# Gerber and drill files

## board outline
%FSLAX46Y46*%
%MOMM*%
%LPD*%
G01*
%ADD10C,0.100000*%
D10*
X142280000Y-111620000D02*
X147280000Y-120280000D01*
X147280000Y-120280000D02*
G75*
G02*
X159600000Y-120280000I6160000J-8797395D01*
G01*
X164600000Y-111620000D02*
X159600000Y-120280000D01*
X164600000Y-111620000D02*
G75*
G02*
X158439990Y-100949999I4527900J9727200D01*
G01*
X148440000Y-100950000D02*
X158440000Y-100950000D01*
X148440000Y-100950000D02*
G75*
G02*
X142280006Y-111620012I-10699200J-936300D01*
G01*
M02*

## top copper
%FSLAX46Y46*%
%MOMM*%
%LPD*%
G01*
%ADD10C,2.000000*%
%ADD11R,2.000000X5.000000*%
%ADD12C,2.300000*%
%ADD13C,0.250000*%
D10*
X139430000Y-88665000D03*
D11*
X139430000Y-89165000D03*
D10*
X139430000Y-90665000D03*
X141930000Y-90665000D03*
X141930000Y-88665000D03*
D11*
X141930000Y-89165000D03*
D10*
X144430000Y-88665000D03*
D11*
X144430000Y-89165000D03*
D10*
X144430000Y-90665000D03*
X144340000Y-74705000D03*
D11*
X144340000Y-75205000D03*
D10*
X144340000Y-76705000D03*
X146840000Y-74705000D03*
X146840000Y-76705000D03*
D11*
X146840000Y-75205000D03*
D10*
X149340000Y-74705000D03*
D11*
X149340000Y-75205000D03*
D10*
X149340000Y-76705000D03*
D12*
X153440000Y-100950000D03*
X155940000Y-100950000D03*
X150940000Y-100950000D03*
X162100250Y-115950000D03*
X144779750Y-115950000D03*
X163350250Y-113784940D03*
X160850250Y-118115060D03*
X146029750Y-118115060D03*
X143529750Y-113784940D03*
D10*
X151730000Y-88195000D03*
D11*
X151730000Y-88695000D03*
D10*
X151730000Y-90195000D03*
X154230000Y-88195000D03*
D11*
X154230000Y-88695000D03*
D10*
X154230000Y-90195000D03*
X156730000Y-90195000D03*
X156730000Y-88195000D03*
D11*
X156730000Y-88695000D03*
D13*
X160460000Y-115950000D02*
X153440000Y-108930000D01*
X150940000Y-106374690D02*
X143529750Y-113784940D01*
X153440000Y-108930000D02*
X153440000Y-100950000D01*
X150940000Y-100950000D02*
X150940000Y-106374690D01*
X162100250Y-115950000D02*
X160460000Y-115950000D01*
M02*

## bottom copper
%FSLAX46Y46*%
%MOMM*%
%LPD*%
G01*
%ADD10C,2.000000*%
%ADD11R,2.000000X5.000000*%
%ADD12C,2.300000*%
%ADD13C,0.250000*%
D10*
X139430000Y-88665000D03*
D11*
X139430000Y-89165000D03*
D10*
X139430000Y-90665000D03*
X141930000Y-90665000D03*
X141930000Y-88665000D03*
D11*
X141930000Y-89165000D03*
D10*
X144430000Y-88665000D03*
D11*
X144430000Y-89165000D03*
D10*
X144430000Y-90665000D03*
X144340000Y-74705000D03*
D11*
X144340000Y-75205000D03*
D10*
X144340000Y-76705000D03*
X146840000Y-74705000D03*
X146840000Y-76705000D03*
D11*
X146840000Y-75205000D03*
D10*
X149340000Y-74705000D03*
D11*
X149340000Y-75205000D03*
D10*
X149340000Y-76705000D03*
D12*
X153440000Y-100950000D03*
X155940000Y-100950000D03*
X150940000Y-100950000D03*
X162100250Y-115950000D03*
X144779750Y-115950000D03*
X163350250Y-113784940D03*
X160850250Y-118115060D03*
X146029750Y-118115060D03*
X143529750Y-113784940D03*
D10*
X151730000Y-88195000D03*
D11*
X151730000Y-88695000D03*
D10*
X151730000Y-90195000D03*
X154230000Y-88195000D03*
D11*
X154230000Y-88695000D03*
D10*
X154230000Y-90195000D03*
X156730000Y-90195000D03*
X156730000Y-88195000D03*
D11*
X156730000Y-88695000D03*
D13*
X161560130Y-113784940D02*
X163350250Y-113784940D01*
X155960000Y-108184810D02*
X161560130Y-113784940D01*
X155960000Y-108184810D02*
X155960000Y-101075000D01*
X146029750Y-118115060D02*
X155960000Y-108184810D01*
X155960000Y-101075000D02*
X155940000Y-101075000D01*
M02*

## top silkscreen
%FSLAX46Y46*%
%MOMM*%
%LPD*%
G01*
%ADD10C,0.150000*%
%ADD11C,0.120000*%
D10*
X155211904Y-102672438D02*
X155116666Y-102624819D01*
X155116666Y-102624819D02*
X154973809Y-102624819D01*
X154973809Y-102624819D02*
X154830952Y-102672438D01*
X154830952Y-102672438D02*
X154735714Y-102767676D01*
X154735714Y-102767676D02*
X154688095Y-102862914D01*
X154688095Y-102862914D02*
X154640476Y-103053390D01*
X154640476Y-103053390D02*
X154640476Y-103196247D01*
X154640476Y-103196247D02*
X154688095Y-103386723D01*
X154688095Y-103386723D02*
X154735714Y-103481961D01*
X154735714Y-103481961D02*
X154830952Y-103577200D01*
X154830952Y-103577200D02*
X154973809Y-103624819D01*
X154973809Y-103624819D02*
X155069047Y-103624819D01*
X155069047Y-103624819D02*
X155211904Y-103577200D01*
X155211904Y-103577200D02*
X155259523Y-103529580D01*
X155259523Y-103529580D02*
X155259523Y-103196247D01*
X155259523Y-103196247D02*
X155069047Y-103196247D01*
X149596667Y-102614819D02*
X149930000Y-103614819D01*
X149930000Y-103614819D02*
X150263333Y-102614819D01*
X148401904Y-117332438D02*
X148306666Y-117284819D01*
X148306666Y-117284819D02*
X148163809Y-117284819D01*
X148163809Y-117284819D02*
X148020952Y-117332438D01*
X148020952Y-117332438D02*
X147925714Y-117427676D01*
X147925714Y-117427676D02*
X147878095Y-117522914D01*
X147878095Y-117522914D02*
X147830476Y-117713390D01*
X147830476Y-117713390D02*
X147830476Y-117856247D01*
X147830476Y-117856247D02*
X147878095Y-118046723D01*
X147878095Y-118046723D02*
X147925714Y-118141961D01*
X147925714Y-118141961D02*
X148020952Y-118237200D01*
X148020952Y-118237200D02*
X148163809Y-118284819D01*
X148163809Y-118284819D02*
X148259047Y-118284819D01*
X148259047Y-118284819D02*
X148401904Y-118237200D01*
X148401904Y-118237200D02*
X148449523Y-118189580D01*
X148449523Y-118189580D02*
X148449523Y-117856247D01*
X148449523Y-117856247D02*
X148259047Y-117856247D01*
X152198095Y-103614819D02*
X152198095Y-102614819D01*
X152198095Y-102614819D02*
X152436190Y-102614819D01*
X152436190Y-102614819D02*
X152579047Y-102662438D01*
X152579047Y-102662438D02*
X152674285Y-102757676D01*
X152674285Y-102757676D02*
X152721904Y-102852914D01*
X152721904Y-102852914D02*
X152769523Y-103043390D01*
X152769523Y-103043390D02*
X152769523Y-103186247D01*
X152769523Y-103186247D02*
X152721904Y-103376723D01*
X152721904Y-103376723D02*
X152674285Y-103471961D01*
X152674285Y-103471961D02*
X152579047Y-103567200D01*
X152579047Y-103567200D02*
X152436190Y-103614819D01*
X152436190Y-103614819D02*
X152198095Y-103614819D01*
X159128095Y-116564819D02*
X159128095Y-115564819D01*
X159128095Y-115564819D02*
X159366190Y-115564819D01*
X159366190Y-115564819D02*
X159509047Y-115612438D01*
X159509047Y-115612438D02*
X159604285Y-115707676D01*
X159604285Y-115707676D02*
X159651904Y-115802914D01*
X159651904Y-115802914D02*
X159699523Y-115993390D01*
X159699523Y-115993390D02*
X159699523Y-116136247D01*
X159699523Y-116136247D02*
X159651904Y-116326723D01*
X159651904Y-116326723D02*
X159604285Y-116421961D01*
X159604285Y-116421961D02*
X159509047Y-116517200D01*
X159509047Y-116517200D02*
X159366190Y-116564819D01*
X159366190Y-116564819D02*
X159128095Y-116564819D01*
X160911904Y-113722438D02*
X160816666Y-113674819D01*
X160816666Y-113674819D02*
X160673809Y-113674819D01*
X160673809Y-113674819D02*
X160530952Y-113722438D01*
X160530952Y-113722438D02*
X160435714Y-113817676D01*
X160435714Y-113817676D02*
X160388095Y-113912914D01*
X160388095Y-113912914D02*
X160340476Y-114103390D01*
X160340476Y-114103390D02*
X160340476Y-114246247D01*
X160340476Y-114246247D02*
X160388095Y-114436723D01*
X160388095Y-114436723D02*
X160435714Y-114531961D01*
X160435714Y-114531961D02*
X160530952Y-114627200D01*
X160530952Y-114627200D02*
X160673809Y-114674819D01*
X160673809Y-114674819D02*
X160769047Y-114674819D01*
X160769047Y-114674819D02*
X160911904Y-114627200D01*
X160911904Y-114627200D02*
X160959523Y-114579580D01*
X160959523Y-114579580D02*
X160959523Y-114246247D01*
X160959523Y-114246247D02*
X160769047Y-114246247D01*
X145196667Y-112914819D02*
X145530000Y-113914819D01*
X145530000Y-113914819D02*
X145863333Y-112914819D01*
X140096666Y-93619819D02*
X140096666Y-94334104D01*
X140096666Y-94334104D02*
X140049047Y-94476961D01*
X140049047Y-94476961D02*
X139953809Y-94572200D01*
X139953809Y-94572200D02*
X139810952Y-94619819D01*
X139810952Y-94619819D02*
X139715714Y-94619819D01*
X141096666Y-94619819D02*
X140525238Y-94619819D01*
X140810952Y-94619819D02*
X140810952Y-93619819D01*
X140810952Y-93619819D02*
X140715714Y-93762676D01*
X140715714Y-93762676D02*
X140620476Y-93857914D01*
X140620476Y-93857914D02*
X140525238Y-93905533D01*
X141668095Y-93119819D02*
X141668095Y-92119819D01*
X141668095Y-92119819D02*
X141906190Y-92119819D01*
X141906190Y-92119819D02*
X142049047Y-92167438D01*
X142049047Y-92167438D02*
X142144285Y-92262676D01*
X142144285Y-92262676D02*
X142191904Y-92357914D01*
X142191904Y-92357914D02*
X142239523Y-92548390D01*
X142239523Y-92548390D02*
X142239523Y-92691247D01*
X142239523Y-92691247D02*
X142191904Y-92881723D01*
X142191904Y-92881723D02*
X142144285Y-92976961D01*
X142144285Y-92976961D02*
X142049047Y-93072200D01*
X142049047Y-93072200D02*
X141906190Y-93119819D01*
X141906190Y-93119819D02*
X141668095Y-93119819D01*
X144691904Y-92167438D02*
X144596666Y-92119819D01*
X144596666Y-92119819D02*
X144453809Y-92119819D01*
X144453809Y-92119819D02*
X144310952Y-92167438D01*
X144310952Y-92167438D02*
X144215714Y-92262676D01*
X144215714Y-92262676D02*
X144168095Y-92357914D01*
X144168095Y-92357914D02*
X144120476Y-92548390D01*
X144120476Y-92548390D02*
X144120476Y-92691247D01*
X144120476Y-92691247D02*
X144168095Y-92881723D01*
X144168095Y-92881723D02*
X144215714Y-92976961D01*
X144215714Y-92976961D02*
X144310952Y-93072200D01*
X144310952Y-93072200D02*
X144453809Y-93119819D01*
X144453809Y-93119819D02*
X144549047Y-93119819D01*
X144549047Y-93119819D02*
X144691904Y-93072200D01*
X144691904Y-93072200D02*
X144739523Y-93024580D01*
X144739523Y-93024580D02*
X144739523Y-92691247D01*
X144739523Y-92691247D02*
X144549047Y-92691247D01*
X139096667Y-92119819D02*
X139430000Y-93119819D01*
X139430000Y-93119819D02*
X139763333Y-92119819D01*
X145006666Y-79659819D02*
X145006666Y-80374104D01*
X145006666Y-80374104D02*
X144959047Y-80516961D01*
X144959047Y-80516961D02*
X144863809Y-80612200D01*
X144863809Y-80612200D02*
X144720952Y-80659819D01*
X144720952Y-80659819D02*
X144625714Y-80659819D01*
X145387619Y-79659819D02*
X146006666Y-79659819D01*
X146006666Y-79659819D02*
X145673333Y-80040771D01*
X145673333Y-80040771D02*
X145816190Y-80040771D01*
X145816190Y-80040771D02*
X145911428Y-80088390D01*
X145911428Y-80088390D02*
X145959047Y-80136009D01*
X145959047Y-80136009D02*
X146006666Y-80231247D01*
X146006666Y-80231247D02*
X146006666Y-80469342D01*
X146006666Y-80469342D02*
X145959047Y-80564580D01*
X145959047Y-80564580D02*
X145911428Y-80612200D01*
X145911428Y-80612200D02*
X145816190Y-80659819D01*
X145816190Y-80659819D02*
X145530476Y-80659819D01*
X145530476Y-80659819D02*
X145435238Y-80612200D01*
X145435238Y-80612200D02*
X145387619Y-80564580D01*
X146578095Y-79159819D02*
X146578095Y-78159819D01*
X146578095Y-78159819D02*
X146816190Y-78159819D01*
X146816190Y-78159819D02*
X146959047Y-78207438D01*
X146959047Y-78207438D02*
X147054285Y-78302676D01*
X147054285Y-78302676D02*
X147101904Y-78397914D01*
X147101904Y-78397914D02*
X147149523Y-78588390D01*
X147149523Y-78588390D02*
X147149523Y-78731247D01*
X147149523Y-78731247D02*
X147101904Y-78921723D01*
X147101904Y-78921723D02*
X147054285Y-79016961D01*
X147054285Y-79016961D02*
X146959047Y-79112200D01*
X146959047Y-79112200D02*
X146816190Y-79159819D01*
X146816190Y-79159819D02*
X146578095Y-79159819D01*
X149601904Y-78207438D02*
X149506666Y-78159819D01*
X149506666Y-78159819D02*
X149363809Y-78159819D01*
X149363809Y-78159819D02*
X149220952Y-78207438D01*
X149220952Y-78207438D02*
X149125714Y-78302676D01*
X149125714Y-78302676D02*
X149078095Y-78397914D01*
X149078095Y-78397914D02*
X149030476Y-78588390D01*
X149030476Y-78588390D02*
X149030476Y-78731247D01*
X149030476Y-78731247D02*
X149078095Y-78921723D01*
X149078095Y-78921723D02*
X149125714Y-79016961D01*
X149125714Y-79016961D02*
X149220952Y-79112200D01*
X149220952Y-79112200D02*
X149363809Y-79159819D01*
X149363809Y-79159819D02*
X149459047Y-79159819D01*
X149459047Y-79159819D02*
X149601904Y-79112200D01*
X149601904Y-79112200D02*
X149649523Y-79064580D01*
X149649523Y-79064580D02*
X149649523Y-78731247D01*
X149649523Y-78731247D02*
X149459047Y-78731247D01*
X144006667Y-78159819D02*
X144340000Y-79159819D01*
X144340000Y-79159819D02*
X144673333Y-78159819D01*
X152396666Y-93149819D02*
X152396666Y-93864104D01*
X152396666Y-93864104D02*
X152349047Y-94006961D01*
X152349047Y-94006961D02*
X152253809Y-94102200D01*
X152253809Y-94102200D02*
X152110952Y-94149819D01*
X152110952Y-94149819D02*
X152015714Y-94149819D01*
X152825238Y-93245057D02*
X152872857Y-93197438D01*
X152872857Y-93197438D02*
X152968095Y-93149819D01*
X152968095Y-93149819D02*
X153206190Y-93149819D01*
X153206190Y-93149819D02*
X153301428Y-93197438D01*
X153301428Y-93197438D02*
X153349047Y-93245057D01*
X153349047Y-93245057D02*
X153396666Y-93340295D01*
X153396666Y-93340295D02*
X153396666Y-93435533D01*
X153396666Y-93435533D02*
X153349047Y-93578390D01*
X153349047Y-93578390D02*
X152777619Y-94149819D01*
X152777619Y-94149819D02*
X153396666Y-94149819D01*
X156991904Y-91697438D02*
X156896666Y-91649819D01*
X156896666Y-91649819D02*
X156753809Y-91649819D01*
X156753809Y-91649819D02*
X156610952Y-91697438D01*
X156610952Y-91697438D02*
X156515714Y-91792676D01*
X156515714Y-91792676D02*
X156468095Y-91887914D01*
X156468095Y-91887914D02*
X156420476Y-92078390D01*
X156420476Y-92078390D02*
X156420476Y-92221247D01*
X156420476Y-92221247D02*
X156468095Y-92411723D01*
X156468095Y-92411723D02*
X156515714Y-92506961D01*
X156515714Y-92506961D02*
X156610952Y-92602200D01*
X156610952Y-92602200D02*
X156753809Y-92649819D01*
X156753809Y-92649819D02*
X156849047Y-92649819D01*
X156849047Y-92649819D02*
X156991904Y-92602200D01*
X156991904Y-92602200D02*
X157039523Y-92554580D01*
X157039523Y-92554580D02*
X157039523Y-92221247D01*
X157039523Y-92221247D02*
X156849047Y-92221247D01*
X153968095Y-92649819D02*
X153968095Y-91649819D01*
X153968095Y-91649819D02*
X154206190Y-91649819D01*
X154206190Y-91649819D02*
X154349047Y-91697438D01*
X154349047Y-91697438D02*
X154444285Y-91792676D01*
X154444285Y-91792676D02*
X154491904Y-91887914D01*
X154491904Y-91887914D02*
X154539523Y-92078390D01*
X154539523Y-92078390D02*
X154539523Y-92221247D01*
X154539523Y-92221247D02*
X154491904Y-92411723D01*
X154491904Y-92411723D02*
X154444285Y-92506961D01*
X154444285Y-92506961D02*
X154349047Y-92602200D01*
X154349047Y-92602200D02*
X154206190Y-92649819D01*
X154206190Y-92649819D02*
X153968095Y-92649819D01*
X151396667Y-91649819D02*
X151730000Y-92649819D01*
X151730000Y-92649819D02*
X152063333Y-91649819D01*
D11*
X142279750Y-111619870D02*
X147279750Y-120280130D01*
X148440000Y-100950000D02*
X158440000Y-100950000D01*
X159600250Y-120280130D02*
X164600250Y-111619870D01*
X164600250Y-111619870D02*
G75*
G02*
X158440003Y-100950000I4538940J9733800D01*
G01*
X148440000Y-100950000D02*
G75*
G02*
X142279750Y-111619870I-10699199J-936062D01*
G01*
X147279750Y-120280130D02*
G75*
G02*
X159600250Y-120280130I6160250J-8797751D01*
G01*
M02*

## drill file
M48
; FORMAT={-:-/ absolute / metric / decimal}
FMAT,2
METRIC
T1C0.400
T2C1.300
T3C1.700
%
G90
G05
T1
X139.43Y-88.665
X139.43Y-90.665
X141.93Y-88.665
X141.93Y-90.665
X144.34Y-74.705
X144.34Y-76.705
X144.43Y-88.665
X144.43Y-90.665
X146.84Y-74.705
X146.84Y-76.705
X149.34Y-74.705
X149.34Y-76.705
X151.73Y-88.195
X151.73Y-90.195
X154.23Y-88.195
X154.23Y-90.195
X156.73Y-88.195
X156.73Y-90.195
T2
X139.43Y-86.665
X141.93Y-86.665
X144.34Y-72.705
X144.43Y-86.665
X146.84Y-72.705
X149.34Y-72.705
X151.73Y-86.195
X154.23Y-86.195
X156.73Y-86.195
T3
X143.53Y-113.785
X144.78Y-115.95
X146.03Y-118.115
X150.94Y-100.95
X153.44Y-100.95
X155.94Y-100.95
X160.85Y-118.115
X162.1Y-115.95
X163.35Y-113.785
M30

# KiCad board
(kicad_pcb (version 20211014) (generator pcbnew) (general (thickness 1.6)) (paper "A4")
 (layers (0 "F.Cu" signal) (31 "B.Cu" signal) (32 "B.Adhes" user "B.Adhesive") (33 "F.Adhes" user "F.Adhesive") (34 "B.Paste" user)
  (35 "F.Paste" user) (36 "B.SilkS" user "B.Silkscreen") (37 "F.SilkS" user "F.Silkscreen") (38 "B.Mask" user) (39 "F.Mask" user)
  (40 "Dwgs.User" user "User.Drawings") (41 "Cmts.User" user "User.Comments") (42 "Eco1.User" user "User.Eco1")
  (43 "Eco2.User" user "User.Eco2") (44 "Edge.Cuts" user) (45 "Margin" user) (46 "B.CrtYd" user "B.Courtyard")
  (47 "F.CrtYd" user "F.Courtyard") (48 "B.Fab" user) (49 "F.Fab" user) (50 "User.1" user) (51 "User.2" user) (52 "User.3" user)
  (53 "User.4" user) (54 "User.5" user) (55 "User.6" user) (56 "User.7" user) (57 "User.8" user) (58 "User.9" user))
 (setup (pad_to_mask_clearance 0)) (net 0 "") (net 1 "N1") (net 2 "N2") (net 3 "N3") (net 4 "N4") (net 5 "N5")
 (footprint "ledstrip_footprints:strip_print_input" (layer "F.Cu") (at 141.93 86.665)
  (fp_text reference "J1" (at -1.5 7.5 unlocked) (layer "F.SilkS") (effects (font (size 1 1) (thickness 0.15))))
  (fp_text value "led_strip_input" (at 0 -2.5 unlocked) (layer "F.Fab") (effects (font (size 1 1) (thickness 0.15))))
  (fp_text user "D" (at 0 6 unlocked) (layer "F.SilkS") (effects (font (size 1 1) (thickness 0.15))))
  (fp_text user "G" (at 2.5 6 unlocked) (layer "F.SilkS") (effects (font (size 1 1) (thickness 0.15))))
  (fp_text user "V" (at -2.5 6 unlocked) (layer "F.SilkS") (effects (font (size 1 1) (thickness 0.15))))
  (pad "1" thru_hole circle (at -2.5 2) (size 2 2) (drill 0.4) (layers *.Cu *.Mask) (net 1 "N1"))
  (pad "1" thru_hole rect (at -2.5 0) (size 2 5) (drill 1.3 (offset 0 2.5)) (layers *.Cu *.Mask) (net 1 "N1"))
  (pad "1" thru_hole circle (at -2.5 4) (size 2 2) (drill 0.4) (layers *.Cu *.Mask) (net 1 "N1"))
  (pad "2" thru_hole circle (at 0 4) (size 2 2) (drill 0.4) (layers *.Cu *.Mask) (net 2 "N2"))
  (pad "2" thru_hole circle (at 0 2) (size 2 2) (drill 0.4) (layers *.Cu *.Mask) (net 2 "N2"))
  (pad "2" thru_hole rect (at 0 0) (size 2 5) (drill 1.3 (offset 0 2.5)) (layers *.Cu *.Mask) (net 2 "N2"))
  (pad "3" thru_hole circle (at 2.5 2) (size 2 2) (drill 0.4) (layers *.Cu *.Mask) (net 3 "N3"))
  (pad "3" thru_hole rect (at 2.5 0) (size 2 5) (drill 1.3 (offset 0 2.5)) (layers *.Cu *.Mask) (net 3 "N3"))
  (pad "3" thru_hole circle (at 2.5 4) (size 2 2) (drill 0.4) (layers *.Cu *.Mask) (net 3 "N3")))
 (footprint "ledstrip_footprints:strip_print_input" (layer "F.Cu") (at 146.84 72.705)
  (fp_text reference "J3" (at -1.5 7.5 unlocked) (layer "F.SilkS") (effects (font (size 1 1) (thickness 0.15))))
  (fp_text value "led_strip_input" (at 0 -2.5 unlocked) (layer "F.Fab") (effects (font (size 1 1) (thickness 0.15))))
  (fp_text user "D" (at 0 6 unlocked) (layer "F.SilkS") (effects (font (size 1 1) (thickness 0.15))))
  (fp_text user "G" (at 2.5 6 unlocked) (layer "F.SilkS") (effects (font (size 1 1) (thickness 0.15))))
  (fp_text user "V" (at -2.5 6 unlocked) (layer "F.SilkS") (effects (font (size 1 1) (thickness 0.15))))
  (pad "1" thru_hole circle (at -2.5 2) (size 2 2) (drill 0.4) (layers *.Cu *.Mask) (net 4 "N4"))
  (pad "1" thru_hole rect (at -2.5 0) (size 2 5) (drill 1.3 (offset 0 2.5)) (layers *.Cu *.Mask) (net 4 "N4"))
  (pad "1" thru_hole circle (at -2.5 4) (size 2 2) (drill 0.4) (layers *.Cu *.Mask) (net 4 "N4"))
  (pad "2" thru_hole circle (at 0 2) (size 2 2) (drill 0.4) (layers *.Cu *.Mask) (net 2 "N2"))
  (pad "2" thru_hole circle (at 0 4) (size 2 2) (drill 0.4) (layers *.Cu *.Mask) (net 2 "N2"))
  (pad "2" thru_hole rect (at 0 0) (size 2 5) (drill 1.3 (offset 0 2.5)) (layers *.Cu *.Mask) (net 2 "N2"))
  (pad "3" thru_hole circle (at 2.5 2) (size 2 2) (drill 0.4) (layers *.Cu *.Mask) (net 3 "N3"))
  (pad "3" thru_hole rect (at 2.5 0) (size 2 5) (drill 1.3 (offset 0 2.5)) (layers *.Cu *.Mask) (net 3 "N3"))
  (pad "3" thru_hole circle (at 2.5 4) (size 2 2) (drill 0.4) (layers *.Cu *.Mask) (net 3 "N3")))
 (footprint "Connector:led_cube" (layer "F.Cu") (at 153.44 110.95)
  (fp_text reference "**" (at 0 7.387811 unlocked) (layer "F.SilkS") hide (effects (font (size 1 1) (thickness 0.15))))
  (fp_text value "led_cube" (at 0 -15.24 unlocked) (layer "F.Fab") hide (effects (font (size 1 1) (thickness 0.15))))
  (fp_line (start -11.16025 0.66987) (end -6.16025 9.33013) (layer "F.SilkS") (width 0.12))
  (fp_line (start -5 -10) (end 5 -10) (layer "F.SilkS") (width 0.12))
  (fp_line (start 6.16025 9.33013) (end 11.16025 0.66987) (layer "F.SilkS") (width 0.12))
  (fp_arc (start 11.16025 0.66987) (mid 6.398025 -3.693904) (end 5 -10) (layer "F.SilkS") (width 0.12))
  (fp_arc (start -5 -10) (mid -6.398026 -3.693905) (end -11.16025 0.66987) (layer "F.SilkS") (width 0.12))
  (fp_arc (start -6.16025 9.33013) (mid 0 7.387811) (end 6.16025 9.33013) (layer "F.SilkS") (width 0.12))
  (pad "1" thru_hole circle (at 0 -10) (size 2.3 2.3) (drill 1.7) (layers F&B.Cu *.Mask))
  (pad "2" thru_hole circle (at 2.5 -10) (size 2.3 2.3) (drill 1.7) (layers F&B.Cu *.Mask))
  (pad "3" thru_hole circle (at -2.5 -10) (size 2.3 2.3) (drill 1.7) (layers F&B.Cu *.Mask))
  (pad "4" thru_hole circle (at 8.66025 5) (size 2.3 2.3) (drill 1.7) (layers F&B.Cu *.Mask))
  (pad "5" thru_hole circle (at -8.66025 5) (size 2.3 2.3) (drill 1.7) (layers F&B.Cu *.Mask))
  (pad "6" thru_hole circle (at 9.91025 2.83494) (size 2.3 2.3) (drill 1.7) (layers F&B.Cu *.Mask))
  (pad "7" thru_hole circle (at 7.41025 7.16506) (size 2.3 2.3) (drill 1.7) (layers F&B.Cu *.Mask))
  (pad "8" thru_hole circle (at -7.41025 7.16506) (size 2.3 2.3) (drill 1.7) (layers F&B.Cu *.Mask))
  (pad "9" thru_hole circle (at -9.91025 2.83494) (size 2.3 2.3) (drill 1.7) (layers F&B.Cu *.Mask)))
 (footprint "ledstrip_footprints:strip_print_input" (layer "F.Cu") (at 154.23 86.195)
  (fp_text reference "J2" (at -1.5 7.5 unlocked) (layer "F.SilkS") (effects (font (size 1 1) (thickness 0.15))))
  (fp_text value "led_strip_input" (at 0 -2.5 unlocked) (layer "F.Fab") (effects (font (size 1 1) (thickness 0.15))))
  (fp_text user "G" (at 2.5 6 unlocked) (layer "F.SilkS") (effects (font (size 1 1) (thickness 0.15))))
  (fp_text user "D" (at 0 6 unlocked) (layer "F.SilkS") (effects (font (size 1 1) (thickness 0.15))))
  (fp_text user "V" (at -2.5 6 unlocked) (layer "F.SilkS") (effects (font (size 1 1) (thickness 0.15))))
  (pad "1" thru_hole circle (at -2.5 2) (size 2 2) (drill 0.4) (layers *.Cu *.Mask) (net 1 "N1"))
  (pad "1" thru_hole rect (at -2.5 0) (size 2 5) (drill 1.3 (offset 0 2.5)) (layers *.Cu *.Mask) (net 1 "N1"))
  (pad "1" thru_hole circle (at -2.5 4) (size 2 2) (drill 0.4) (layers *.Cu *.Mask) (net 1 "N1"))
  (pad "2" thru_hole circle (at 0 2) (size 2 2) (drill 0.4) (layers *.Cu *.Mask) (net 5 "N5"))
  (pad "2" thru_hole rect (at 0 0) (size 2 5) (drill 1.3 (offset 0 2.5)) (layers *.Cu *.Mask) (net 5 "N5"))
  (pad "2" thru_hole circle (at 0 4) (size 2 2) (drill 0.4) (layers *.Cu *.Mask) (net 5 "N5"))
  (pad "3" thru_hole circle (at 2.5 4) (size 2 2) (drill 0.4) (layers *.Cu *.Mask) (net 3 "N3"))
  (pad "3" thru_hole circle (at 2.5 2) (size 2 2) (drill 0.4) (layers *.Cu *.Mask) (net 3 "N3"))
  (pad "3" thru_hole rect (at 2.5 0) (size 2 5) (drill 1.3 (offset 0 2.5)) (layers *.Cu *.Mask) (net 3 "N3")))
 (gr_line (start 142.28 111.62) (end 147.28 120.28) (layer "Edge.Cuts") (width 0.1))
 (gr_arc (start 147.28 120.28) (mid 153.44 118.33776) (end 159.6 120.28) (layer "Edge.Cuts") (width 0.1))
 (gr_line (start 164.6 111.62) (end 159.6 120.28) (layer "Edge.Cuts") (width 0.1))
 (gr_arc (start 164.6 111.62) (mid 159.835832 107.257303) (end 158.44 100.95) (layer "Edge.Cuts") (width 0.1))
 (gr_line (start 148.44 100.95) (end 158.44 100.95) (layer "Edge.Cuts") (width 0.1))
 (gr_arc (start 148.44 100.95) (mid 147.04212 107.256121) (end 142.28 111.62) (layer "Edge.Cuts") (width 0.1))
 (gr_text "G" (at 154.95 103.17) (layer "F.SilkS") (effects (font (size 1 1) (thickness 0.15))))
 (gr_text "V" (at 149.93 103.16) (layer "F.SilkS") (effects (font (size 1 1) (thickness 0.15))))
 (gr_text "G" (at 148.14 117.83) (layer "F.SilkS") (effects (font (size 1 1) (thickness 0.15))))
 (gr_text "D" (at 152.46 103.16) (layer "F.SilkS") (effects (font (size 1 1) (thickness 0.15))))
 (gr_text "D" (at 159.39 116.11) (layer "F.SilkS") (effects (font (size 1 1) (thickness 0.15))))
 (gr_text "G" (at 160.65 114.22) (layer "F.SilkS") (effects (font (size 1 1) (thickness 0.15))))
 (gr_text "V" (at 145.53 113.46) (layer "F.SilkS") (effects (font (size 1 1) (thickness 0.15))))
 (segment (start 160.46 115.95) (end 153.44 108.93) (width 0.25) (layer "F.Cu") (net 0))
 (segment (start 150.94 106.37469) (end 143.52975 113.78494) (width 0.25) (layer "F.Cu") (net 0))
 (segment (start 153.44 108.93) (end 153.44 100.95) (width 0.25) (layer "F.Cu") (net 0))
 (segment (start 150.94 100.95) (end 150.94 106.37469) (width 0.25) (layer "F.Cu") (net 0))
 (segment (start 162.10025 115.95) (end 160.46 115.95) (width 0.25) (layer "F.Cu") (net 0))
 (segment (start 161.56013 113.78494) (end 163.35025 113.78494) (width 0.25) (layer "B.Cu") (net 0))
 (segment (start 155.96 108.18481) (end 161.56013 113.78494) (width 0.25) (layer "B.Cu") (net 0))
 (segment (start 155.96 108.18481) (end 155.96 101.075) (width 0.25) (layer "B.Cu") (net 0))
 (segment (start 146.02975 118.11506) (end 155.96 108.18481) (width 0.25) (layer "B.Cu") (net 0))
 (segment (start 155.96 101.075) (end 155.94 101.075) (width 0.25) (layer "B.Cu") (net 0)))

